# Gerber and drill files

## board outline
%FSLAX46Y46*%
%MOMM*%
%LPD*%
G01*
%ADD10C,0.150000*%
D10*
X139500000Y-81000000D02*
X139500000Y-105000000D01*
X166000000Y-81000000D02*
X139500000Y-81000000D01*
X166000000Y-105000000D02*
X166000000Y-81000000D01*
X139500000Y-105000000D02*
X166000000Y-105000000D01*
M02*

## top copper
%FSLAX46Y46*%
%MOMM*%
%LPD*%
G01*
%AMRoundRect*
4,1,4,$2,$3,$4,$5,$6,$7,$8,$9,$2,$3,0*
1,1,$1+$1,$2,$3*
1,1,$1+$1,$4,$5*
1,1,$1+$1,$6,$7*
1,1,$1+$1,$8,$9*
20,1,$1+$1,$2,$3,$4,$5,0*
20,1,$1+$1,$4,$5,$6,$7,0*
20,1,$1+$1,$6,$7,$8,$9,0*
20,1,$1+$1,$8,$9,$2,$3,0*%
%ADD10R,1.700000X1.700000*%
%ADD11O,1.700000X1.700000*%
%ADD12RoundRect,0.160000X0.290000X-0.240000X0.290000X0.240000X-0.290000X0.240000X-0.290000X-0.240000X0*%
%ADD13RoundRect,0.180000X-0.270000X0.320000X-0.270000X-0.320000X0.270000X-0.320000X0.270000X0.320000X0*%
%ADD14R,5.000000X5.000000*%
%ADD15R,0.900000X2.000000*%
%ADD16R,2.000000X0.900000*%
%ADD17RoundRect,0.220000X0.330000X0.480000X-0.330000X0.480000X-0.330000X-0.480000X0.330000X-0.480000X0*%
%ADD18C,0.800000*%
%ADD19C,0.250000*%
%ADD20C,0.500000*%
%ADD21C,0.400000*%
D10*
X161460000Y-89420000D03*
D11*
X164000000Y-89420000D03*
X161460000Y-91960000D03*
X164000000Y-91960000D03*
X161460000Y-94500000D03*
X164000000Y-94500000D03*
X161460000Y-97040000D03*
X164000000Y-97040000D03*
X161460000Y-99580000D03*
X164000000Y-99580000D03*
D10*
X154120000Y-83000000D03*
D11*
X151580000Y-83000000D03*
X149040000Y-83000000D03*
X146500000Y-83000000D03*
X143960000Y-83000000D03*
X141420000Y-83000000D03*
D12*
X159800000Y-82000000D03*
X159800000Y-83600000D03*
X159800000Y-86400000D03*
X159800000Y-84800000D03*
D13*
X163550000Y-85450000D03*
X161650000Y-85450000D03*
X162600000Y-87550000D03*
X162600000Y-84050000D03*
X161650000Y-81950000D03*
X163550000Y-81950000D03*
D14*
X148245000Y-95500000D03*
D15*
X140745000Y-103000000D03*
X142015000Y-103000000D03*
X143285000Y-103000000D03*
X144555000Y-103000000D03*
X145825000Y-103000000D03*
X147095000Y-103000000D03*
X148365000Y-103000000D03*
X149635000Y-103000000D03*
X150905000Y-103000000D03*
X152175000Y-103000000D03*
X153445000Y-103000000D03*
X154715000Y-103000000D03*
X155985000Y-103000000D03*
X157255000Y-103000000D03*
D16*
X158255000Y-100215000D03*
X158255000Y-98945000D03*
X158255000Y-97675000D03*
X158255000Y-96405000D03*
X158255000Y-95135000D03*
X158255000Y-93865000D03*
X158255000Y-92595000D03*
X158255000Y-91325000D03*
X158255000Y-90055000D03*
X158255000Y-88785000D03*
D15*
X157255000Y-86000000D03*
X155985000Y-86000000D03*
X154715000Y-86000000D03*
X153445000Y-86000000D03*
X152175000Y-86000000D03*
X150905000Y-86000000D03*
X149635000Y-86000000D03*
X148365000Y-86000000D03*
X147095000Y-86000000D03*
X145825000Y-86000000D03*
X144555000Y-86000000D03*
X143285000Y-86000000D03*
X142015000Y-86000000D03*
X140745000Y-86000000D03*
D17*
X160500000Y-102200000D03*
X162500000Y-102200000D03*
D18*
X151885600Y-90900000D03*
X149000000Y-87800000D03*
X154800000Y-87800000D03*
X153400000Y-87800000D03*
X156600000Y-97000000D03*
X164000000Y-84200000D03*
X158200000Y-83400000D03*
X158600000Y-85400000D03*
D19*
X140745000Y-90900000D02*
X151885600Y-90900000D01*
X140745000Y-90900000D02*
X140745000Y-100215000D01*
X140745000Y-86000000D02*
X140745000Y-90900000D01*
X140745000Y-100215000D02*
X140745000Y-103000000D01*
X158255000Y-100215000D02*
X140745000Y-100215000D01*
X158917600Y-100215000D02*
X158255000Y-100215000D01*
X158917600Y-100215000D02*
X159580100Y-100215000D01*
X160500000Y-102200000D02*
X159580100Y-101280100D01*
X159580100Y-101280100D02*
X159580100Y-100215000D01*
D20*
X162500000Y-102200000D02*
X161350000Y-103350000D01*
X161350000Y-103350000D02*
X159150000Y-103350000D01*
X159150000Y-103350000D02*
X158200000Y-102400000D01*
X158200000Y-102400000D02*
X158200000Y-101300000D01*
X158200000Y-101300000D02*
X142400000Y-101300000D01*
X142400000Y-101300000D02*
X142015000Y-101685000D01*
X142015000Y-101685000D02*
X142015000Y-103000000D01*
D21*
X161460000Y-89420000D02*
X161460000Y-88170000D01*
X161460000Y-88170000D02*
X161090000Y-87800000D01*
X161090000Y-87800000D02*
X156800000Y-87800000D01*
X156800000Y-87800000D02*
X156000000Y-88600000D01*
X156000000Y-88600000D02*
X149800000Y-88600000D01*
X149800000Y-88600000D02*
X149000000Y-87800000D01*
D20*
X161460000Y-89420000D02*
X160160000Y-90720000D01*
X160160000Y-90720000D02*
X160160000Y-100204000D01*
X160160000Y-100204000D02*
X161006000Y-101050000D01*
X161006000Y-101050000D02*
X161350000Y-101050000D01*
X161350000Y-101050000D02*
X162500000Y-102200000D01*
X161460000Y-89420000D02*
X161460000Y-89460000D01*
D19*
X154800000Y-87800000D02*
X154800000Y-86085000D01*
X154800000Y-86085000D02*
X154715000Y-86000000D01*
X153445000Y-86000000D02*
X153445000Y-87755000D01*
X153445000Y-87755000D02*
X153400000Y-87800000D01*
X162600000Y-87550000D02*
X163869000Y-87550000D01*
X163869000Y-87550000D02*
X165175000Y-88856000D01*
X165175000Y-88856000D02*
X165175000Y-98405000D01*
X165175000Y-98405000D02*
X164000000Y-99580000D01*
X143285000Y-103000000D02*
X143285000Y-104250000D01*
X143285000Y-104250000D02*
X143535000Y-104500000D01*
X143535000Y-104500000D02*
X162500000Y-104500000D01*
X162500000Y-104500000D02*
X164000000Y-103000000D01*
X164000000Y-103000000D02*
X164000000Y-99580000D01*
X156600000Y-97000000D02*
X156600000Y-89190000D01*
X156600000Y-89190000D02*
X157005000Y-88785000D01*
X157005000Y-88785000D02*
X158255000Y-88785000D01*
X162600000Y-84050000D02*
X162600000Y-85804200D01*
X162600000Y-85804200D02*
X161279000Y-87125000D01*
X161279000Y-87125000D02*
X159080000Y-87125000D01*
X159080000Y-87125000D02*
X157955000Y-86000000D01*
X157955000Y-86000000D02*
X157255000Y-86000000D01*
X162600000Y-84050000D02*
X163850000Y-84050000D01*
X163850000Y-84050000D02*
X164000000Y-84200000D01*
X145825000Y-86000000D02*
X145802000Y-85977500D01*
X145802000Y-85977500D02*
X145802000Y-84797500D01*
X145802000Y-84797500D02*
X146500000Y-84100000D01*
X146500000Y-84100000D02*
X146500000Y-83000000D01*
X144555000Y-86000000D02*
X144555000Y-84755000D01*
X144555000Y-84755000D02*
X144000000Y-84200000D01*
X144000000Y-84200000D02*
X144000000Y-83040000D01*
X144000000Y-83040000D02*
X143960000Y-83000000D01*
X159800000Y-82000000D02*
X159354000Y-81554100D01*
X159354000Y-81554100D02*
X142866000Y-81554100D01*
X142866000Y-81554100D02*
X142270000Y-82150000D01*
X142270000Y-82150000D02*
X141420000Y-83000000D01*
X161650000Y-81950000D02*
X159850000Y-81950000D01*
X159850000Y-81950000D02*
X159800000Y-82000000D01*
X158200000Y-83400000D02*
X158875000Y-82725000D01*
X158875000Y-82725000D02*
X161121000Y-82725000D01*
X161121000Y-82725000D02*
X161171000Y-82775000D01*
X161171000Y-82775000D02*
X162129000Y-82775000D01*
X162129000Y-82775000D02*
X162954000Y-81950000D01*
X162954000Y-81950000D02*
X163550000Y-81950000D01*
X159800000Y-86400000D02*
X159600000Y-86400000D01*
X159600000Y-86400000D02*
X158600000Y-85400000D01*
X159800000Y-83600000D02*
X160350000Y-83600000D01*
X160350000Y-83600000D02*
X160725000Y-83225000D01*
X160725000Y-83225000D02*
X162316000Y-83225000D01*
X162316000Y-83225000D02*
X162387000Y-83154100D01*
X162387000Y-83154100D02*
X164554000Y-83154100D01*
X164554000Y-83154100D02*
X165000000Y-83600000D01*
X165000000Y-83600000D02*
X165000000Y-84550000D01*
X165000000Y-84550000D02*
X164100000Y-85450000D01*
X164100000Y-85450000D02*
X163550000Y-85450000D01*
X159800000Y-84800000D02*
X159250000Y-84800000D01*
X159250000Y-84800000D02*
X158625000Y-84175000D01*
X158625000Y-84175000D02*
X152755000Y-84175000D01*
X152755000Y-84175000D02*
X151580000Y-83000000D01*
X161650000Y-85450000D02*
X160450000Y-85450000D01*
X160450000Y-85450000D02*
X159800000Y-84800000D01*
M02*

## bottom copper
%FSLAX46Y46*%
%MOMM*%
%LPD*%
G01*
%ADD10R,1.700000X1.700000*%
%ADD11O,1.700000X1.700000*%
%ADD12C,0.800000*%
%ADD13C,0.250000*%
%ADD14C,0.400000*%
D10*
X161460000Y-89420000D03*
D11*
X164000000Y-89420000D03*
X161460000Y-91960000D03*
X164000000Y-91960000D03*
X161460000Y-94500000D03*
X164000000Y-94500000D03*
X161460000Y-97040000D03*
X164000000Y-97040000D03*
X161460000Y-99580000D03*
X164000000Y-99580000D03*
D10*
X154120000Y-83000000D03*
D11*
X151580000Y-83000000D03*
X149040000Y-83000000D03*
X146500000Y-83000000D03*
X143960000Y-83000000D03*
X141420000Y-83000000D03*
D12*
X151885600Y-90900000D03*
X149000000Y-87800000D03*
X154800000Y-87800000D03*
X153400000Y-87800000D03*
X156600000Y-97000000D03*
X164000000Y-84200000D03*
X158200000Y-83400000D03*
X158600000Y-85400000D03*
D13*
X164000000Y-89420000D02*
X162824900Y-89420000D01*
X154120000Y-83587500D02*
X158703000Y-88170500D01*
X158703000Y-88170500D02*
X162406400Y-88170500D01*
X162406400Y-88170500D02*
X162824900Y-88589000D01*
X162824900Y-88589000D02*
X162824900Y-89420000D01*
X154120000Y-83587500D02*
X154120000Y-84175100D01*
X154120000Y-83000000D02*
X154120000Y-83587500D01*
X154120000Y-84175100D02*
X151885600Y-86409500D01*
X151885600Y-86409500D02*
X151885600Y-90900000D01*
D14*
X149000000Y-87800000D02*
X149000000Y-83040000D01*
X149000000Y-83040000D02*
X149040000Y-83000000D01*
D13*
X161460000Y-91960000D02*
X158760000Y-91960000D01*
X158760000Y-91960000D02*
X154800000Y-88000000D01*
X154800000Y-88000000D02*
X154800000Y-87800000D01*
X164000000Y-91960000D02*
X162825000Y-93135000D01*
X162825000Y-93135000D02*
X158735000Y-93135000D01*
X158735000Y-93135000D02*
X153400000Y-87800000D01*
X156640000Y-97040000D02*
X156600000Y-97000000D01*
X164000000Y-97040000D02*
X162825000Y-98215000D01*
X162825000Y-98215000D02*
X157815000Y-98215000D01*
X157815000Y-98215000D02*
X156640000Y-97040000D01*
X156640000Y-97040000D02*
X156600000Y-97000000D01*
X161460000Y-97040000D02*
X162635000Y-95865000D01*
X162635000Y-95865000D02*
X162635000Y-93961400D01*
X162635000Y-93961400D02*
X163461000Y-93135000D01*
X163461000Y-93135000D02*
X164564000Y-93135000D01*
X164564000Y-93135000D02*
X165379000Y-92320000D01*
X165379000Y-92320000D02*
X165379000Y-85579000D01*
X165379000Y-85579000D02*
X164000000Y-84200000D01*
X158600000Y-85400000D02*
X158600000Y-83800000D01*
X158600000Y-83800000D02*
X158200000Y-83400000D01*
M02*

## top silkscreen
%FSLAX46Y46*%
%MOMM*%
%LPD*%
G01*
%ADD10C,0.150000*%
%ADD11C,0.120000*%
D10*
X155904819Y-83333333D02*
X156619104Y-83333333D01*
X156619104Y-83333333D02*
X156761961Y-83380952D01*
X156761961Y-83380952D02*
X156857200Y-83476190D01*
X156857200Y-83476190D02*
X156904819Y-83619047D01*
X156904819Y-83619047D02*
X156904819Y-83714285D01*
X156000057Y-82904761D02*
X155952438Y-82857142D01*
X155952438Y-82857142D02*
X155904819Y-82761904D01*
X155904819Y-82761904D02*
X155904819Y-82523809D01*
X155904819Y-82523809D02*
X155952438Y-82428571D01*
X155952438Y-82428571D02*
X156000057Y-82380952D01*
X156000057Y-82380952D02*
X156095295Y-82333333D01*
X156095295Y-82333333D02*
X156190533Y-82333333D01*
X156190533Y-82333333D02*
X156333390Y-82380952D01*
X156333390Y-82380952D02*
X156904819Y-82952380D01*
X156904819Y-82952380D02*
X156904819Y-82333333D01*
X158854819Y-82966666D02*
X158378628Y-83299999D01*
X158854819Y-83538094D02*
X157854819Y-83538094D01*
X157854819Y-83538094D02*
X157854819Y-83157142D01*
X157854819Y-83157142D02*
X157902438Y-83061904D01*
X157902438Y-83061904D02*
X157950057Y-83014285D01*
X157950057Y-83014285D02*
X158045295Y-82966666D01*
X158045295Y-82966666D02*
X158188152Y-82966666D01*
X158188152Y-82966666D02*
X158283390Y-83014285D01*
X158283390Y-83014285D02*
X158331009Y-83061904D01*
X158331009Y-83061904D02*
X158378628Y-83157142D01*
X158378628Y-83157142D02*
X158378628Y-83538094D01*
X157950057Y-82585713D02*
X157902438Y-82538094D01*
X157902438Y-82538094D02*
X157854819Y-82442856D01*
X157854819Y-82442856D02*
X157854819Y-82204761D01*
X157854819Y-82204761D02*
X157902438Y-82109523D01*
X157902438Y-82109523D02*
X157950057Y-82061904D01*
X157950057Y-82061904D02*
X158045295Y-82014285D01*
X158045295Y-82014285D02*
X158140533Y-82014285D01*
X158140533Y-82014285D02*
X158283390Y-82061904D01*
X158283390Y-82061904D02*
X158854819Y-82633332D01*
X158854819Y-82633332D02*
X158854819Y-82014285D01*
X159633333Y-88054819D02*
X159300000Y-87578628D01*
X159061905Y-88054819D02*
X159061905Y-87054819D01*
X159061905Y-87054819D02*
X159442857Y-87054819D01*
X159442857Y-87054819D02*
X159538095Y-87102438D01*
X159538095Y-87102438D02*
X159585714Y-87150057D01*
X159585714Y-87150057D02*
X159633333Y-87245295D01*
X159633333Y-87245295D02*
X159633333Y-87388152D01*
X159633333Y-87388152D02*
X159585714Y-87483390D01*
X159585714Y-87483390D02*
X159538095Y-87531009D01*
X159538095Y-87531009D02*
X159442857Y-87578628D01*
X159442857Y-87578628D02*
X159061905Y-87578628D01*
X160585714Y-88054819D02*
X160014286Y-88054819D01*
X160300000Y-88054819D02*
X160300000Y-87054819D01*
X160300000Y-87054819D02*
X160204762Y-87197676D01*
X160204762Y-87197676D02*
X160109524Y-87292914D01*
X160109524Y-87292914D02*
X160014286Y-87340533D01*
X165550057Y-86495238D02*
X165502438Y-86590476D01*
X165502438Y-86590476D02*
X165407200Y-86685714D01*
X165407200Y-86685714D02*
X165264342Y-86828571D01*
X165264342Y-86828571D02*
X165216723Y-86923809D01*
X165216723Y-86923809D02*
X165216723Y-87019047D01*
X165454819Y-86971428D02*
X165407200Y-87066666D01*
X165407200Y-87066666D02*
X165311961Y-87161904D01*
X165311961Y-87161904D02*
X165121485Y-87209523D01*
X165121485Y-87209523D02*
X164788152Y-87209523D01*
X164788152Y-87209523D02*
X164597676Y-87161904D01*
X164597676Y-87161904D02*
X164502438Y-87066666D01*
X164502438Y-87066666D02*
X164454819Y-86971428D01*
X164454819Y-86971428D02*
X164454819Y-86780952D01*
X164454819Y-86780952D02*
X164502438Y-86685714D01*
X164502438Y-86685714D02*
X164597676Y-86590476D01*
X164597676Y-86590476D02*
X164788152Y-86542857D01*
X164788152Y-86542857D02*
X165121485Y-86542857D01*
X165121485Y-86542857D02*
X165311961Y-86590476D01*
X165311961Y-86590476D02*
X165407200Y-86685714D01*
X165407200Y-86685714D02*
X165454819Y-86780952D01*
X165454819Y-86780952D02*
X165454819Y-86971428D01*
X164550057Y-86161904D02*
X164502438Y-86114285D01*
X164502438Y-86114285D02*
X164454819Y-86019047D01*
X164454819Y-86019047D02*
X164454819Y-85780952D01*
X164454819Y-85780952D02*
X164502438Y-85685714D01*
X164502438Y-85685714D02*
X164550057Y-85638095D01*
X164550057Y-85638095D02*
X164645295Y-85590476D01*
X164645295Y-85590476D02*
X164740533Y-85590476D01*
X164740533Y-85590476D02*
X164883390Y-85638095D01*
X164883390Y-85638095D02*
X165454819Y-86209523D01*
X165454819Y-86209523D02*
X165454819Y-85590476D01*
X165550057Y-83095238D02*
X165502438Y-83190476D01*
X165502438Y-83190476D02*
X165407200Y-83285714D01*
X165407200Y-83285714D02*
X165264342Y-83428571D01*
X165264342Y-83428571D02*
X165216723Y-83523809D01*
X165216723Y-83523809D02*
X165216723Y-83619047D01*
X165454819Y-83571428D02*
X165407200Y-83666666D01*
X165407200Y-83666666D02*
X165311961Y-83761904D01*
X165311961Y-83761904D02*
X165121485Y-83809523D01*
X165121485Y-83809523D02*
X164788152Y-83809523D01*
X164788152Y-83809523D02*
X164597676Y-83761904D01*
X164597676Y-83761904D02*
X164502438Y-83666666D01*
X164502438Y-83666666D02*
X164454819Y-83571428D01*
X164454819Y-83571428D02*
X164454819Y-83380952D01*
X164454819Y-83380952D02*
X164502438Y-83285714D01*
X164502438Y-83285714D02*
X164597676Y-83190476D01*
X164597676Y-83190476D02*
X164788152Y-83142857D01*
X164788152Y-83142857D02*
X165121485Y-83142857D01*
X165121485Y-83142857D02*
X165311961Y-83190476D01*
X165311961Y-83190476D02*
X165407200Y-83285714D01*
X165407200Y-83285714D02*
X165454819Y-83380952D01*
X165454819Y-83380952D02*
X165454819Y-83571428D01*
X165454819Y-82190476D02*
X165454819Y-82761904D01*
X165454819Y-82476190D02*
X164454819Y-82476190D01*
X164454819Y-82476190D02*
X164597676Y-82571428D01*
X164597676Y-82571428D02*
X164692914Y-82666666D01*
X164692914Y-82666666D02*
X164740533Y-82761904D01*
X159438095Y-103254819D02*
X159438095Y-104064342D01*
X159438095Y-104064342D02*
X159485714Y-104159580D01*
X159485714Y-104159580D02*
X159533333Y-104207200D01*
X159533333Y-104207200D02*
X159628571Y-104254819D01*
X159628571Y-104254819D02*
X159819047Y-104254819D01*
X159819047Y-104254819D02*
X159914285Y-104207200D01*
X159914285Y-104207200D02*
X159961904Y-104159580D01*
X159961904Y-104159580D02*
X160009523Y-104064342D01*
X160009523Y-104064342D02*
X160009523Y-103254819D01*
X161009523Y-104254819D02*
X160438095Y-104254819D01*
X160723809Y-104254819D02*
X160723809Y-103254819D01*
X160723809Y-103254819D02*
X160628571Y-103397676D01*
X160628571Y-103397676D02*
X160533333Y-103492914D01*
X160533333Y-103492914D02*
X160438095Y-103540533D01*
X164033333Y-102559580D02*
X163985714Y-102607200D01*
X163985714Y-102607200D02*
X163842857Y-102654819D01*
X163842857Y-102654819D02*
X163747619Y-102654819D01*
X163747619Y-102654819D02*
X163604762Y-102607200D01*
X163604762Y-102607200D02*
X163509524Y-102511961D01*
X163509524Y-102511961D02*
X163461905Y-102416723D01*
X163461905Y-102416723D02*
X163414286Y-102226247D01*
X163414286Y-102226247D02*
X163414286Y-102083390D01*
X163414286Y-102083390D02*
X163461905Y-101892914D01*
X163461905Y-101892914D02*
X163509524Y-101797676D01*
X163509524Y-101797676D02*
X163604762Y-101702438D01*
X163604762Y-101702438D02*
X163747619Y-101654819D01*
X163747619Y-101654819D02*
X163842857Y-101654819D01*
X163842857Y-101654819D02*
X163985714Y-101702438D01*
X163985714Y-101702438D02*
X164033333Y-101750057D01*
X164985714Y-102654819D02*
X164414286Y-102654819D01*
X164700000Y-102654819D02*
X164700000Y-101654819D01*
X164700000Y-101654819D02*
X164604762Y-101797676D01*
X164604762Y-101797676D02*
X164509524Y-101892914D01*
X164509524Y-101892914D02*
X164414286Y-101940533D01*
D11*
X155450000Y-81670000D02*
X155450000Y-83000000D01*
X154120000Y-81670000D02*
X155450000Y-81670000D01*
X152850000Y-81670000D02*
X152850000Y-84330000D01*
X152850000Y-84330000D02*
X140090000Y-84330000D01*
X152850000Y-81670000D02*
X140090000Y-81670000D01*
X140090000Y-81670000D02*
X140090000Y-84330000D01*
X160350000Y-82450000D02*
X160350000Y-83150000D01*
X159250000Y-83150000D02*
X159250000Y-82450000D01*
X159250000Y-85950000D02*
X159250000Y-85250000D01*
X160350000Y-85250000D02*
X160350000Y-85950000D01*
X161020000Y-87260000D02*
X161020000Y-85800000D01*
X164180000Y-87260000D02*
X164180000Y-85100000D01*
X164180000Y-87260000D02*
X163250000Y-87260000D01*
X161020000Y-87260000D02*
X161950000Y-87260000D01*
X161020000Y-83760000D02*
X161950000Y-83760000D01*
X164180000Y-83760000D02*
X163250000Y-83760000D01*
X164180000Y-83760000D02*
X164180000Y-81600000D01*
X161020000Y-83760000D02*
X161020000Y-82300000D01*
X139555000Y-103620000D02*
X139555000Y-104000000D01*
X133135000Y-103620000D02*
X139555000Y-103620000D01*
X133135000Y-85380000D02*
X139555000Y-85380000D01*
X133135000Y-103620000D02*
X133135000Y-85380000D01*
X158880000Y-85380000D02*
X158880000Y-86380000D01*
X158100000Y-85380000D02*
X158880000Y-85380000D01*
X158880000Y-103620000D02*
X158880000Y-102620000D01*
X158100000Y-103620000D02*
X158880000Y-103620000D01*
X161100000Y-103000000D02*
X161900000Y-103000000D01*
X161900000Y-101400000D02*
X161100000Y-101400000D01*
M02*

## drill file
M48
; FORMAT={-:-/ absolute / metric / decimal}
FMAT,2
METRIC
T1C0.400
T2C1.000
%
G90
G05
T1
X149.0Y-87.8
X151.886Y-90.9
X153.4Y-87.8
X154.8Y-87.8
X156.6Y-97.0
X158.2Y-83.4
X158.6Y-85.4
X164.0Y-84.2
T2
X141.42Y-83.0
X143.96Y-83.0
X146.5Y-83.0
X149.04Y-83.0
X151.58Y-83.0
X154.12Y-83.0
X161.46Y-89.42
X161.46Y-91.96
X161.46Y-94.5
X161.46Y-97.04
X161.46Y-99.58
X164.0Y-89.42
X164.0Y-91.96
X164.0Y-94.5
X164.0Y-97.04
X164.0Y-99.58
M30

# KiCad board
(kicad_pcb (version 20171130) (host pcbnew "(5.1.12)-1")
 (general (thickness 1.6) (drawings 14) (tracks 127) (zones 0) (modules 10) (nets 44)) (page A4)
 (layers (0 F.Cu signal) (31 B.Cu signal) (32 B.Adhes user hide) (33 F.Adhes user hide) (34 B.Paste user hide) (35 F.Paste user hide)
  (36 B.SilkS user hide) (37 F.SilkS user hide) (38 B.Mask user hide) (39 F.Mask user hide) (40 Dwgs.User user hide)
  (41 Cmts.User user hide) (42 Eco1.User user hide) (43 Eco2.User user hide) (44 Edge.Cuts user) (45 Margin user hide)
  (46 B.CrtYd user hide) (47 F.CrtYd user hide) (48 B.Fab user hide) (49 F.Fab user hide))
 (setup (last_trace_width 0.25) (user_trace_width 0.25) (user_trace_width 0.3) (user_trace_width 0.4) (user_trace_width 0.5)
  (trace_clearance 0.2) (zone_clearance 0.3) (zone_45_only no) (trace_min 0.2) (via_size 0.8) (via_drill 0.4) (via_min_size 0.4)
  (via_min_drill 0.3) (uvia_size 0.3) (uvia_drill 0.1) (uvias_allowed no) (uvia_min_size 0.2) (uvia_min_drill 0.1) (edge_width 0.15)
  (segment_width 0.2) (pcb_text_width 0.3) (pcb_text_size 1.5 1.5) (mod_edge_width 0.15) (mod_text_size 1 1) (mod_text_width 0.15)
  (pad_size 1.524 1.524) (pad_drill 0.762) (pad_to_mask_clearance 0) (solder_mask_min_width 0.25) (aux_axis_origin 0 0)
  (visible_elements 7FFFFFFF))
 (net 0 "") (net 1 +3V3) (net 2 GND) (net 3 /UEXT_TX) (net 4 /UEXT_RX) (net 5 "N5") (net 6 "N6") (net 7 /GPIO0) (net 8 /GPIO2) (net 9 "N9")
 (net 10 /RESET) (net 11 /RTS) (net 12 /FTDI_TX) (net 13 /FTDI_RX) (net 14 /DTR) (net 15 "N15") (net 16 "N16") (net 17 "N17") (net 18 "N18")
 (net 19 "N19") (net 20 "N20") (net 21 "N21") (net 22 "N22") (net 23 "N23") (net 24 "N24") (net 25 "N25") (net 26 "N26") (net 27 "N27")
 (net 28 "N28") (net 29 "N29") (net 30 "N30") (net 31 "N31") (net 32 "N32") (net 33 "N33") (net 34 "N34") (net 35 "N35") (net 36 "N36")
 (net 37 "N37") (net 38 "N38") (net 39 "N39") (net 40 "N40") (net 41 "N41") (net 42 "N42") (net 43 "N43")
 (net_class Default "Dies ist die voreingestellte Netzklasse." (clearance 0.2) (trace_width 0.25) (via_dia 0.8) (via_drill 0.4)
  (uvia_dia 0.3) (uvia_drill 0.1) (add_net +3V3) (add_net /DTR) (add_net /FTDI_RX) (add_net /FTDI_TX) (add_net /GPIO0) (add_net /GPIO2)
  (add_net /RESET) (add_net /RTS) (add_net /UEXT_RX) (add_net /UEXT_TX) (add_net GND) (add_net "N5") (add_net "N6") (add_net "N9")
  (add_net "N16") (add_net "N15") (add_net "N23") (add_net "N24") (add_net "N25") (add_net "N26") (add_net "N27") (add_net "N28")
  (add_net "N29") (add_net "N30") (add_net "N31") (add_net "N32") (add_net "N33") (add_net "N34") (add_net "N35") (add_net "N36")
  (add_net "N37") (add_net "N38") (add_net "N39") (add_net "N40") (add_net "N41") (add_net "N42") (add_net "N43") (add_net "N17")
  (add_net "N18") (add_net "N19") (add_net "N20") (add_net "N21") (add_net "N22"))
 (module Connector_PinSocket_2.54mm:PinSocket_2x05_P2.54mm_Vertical (layer B.Cu) (at 161.46 89.42 180)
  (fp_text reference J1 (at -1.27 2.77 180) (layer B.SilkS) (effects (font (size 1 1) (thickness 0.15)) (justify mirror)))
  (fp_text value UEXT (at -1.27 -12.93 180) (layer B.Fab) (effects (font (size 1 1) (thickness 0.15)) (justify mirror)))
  (pad 1 thru_hole rect (at 0 0 180) (size 1.7 1.7) (drill 1) (layers *.Cu *.Mask) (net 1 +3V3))
  (pad 2 thru_hole oval (at -2.54 0 180) (size 1.7 1.7) (drill 1) (layers *.Cu *.Mask) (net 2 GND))
  (pad 3 thru_hole oval (at 0 -2.54 180) (size 1.7 1.7) (drill 1) (layers *.Cu *.Mask) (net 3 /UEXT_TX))
  (pad 4 thru_hole oval (at -2.54 -2.54 180) (size 1.7 1.7) (drill 1) (layers *.Cu *.Mask) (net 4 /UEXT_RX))
  (pad 5 thru_hole oval (at 0 -5.08 180) (size 1.7 1.7) (drill 1) (layers *.Cu *.Mask) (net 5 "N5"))
  (pad 6 thru_hole oval (at -2.54 -5.08 180) (size 1.7 1.7) (drill 1) (layers *.Cu *.Mask) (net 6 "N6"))
  (pad 7 thru_hole oval (at 0 -7.62 180) (size 1.7 1.7) (drill 1) (layers *.Cu *.Mask) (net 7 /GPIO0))
  (pad 8 thru_hole oval (at -2.54 -7.62 180) (size 1.7 1.7) (drill 1) (layers *.Cu *.Mask) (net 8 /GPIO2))
  (pad 9 thru_hole oval (at 0 -10.16 180) (size 1.7 1.7) (drill 1) (layers *.Cu *.Mask) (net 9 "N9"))
  (pad 10 thru_hole oval (at -2.54 -10.16 180) (size 1.7 1.7) (drill 1) (layers *.Cu *.Mask) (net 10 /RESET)))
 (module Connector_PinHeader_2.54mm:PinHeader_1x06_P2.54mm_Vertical (layer F.Cu) (at 154.12 83 270)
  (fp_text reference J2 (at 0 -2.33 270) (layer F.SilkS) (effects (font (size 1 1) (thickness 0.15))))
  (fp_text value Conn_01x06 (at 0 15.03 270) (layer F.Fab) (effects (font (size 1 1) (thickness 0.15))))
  (fp_line (start -1.33 -1.33) (end 0 -1.33) (layer F.SilkS) (width 0.12))
  (fp_line (start -1.33 0) (end -1.33 -1.33) (layer F.SilkS) (width 0.12))
  (fp_line (start -1.33 1.27) (end 1.33 1.27) (layer F.SilkS) (width 0.12))
  (fp_line (start 1.33 1.27) (end 1.33 14.03) (layer F.SilkS) (width 0.12))
  (fp_line (start -1.33 1.27) (end -1.33 14.03) (layer F.SilkS) (width 0.12))
  (fp_line (start -1.33 14.03) (end 1.33 14.03) (layer F.SilkS) (width 0.12))
  (pad 1 thru_hole rect (at 0 0 270) (size 1.7 1.7) (drill 1) (layers *.Cu *.Mask) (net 2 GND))
  (pad 2 thru_hole oval (at 0 2.54 270) (size 1.7 1.7) (drill 1) (layers *.Cu *.Mask) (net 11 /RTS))
  (pad 3 thru_hole oval (at 0 5.08 270) (size 1.7 1.7) (drill 1) (layers *.Cu *.Mask) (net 1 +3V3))
  (pad 4 thru_hole oval (at 0 7.62 270) (size 1.7 1.7) (drill 1) (layers *.Cu *.Mask) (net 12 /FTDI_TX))
  (pad 5 thru_hole oval (at 0 10.16 270) (size 1.7 1.7) (drill 1) (layers *.Cu *.Mask) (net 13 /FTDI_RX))
  (pad 6 thru_hole oval (at 0 12.7 270) (size 1.7 1.7) (drill 1) (layers *.Cu *.Mask) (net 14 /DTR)))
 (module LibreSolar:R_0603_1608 (layer F.Cu) (at 159.8 82.8 90)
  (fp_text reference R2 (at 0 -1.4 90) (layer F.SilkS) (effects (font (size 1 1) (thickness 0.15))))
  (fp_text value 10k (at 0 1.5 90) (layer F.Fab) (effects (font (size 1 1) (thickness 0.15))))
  (fp_line (start 0.35 0.55) (end -0.35 0.55) (layer F.SilkS) (width 0.12))
  (fp_line (start -0.35 -0.55) (end 0.35 -0.55) (layer F.SilkS) (width 0.12))
  (pad 2 smd roundrect (at 0.8 0 90) (size 0.8 0.9) (layers F.Cu F.Paste F.Mask) (roundrect_rratio 0.2) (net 14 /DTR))
  (pad 1 smd roundrect (at -0.8 0 90) (size 0.8 0.9) (layers F.Cu F.Paste F.Mask) (roundrect_rratio 0.2) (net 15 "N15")))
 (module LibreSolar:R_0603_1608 (layer F.Cu) (at 159.8 85.6 90)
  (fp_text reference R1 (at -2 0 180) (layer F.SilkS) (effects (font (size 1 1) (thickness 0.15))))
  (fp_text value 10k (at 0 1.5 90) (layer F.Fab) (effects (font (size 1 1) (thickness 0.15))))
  (fp_line (start -0.35 -0.55) (end 0.35 -0.55) (layer F.SilkS) (width 0.12))
  (fp_line (start 0.35 0.55) (end -0.35 0.55) (layer F.SilkS) (width 0.12))
  (pad 1 smd roundrect (at -0.8 0 90) (size 0.8 0.9) (layers F.Cu F.Paste F.Mask) (roundrect_rratio 0.2) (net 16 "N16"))
  (pad 2 smd roundrect (at 0.8 0 90) (size 0.8 0.9) (layers F.Cu F.Paste F.Mask) (roundrect_rratio 0.2) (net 11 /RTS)))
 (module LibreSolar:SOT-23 (layer F.Cu) (at 162.6 86.5 270)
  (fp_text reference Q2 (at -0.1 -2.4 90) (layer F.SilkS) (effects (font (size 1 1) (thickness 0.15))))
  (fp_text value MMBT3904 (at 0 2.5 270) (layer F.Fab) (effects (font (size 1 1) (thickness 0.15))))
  (fp_line (start 0.76 1.58) (end -0.7 1.58) (layer F.SilkS) (width 0.12))
  (fp_line (start 0.76 -1.58) (end -1.4 -1.58) (layer F.SilkS) (width 0.12))
  (fp_line (start 0.76 -1.58) (end 0.76 -0.65) (layer F.SilkS) (width 0.12))
  (fp_line (start 0.76 1.58) (end 0.76 0.65) (layer F.SilkS) (width 0.12))
  (pad 1 smd roundrect (at -1.05 -0.95 270) (size 1 0.9) (layers F.Cu F.Paste F.Mask) (roundrect_rratio 0.2) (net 15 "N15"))
  (pad 2 smd roundrect (at -1.05 0.95 270) (size 1 0.9) (layers F.Cu F.Paste F.Mask) (roundrect_rratio 0.2) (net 11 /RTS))
  (pad 3 smd roundrect (at 1.05 0 270) (size 1 0.9) (layers F.Cu F.Paste F.Mask) (roundrect_rratio 0.2) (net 10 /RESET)))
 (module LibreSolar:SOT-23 (layer F.Cu) (at 162.6 83 270)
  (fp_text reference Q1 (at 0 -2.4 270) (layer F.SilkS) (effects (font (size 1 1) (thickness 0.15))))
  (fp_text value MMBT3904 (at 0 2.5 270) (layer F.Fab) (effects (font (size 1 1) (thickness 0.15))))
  (fp_line (start 0.76 1.58) (end 0.76 0.65) (layer F.SilkS) (width 0.12))
  (fp_line (start 0.76 -1.58) (end 0.76 -0.65) (layer F.SilkS) (width 0.12))
  (fp_line (start 0.76 -1.58) (end -1.4 -1.58) (layer F.SilkS) (width 0.12))
  (fp_line (start 0.76 1.58) (end -0.7 1.58) (layer F.SilkS) (width 0.12))
  (pad 3 smd roundrect (at 1.05 0 270) (size 1 0.9) (layers F.Cu F.Paste F.Mask) (roundrect_rratio 0.2) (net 7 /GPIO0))
  (pad 2 smd roundrect (at -1.05 0.95 270) (size 1 0.9) (layers F.Cu F.Paste F.Mask) (roundrect_rratio 0.2) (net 14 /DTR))
  (pad 1 smd roundrect (at -1.05 -0.95 270) (size 1 0.9) (layers F.Cu F.Paste F.Mask) (roundrect_rratio 0.2) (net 16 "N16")))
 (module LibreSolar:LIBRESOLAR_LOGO (layer B.Cu) (at 156 98 180)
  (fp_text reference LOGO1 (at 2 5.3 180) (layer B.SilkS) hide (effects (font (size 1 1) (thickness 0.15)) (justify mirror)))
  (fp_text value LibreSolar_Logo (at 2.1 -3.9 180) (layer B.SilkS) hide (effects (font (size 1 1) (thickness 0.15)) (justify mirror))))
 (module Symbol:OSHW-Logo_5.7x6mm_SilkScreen (layer B.Cu) (at 145.4 97 180)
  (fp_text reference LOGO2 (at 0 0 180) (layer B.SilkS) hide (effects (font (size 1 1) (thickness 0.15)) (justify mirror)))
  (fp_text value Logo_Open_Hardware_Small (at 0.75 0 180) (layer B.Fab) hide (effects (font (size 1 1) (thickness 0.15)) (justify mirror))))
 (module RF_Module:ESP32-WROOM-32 (layer F.Cu) (at 149 94.5 90)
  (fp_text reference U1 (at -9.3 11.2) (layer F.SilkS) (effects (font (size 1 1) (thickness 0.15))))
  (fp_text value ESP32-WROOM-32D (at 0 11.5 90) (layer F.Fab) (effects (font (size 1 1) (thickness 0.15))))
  (fp_line (start -9.12 -9.445) (end -9.5 -9.445) (layer F.SilkS) (width 0.12))
  (fp_line (start -9.12 -15.865) (end -9.12 -9.445) (layer F.SilkS) (width 0.12))
  (fp_line (start 9.12 -15.865) (end 9.12 -9.445) (layer F.SilkS) (width 0.12))
  (fp_line (start -9.12 -15.865) (end 9.12 -15.865) (layer F.SilkS) (width 0.12))
  (fp_line (start 9.12 9.88) (end 8.12 9.88) (layer F.SilkS) (width 0.12))
  (fp_line (start 9.12 9.1) (end 9.12 9.88) (layer F.SilkS) (width 0.12))
  (fp_line (start -9.12 9.88) (end -8.12 9.88) (layer F.SilkS) (width 0.12))
  (fp_line (start -9.12 9.1) (end -9.12 9.88) (layer F.SilkS) (width 0.12))
  (pad 39 smd rect (at -1 -0.755 90) (size 5 5) (layers F.Cu F.Paste F.Mask))
  (pad 1 smd rect (at -8.5 -8.255 90) (size 2 0.9) (layers F.Cu F.Paste F.Mask) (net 2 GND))
  (pad 2 smd rect (at -8.5 -6.985 90) (size 2 0.9) (layers F.Cu F.Paste F.Mask) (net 1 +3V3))
  (pad 3 smd rect (at -8.5 -5.715 90) (size 2 0.9) (layers F.Cu F.Paste F.Mask) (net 10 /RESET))
  (pad 4 smd rect (at -8.5 -4.445 90) (size 2 0.9) (layers F.Cu F.Paste F.Mask) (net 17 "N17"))
  (pad 5 smd rect (at -8.5 -3.175 90) (size 2 0.9) (layers F.Cu F.Paste F.Mask) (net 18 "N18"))
  (pad 6 smd rect (at -8.5 -1.905 90) (size 2 0.9) (layers F.Cu F.Paste F.Mask) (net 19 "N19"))
  (pad 7 smd rect (at -8.5 -0.635 90) (size 2 0.9) (layers F.Cu F.Paste F.Mask) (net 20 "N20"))
  (pad 8 smd rect (at -8.5 0.635 90) (size 2 0.9) (layers F.Cu F.Paste F.Mask) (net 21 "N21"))
  (pad 9 smd rect (at -8.5 1.905 90) (size 2 0.9) (layers F.Cu F.Paste F.Mask) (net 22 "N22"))
  (pad 10 smd rect (at -8.5 3.175 90) (size 2 0.9) (layers F.Cu F.Paste F.Mask) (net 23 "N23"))
  (pad 11 smd rect (at -8.5 4.445 90) (size 2 0.9) (layers F.Cu F.Paste F.Mask) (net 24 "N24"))
  (pad 12 smd rect (at -8.5 5.715 90) (size 2 0.9) (layers F.Cu F.Paste F.Mask) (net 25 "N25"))
  (pad 13 smd rect (at -8.5 6.985 90) (size 2 0.9) (layers F.Cu F.Paste F.Mask) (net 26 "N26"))
  (pad 14 smd rect (at -8.5 8.255 90) (size 2 0.9) (layers F.Cu F.Paste F.Mask) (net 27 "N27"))
  (pad 15 smd rect (at -5.715 9.255 180) (size 2 0.9) (layers F.Cu F.Paste F.Mask) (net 2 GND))
  (pad 16 smd rect (at -4.445 9.255 180) (size 2 0.9) (layers F.Cu F.Paste F.Mask) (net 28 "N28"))
  (pad 17 smd rect (at -3.175 9.255 180) (size 2 0.9) (layers F.Cu F.Paste F.Mask) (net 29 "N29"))
  (pad 18 smd rect (at -1.905 9.255 180) (size 2 0.9) (layers F.Cu F.Paste F.Mask) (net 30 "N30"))
  (pad 19 smd rect (at -0.635 9.255 180) (size 2 0.9) (layers F.Cu F.Paste F.Mask) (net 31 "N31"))
  (pad 20 smd rect (at 0.635 9.255 180) (size 2 0.9) (layers F.Cu F.Paste F.Mask) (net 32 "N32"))
  (pad 21 smd rect (at 1.905 9.255 180) (size 2 0.9) (layers F.Cu F.Paste F.Mask) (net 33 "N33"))
  (pad 22 smd rect (at 3.175 9.255 180) (size 2 0.9) (layers F.Cu F.Paste F.Mask) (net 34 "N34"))
  (pad 23 smd rect (at 4.445 9.255 180) (size 2 0.9) (layers F.Cu F.Paste F.Mask) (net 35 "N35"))
  (pad 24 smd rect (at 5.715 9.255 180) (size 2 0.9) (layers F.Cu F.Paste F.Mask) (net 8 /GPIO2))
  (pad 25 smd rect (at 8.5 8.255 90) (size 2 0.9) (layers F.Cu F.Paste F.Mask) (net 7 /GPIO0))
  (pad 26 smd rect (at 8.5 6.985 90) (size 2 0.9) (layers F.Cu F.Paste F.Mask) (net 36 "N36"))
  (pad 27 smd rect (at 8.5 5.715 90) (size 2 0.9) (layers F.Cu F.Paste F.Mask) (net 3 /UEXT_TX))
  (pad 28 smd rect (at 8.5 4.445 90) (size 2 0.9) (layers F.Cu F.Paste F.Mask) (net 4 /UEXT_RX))
  (pad 29 smd rect (at 8.5 3.175 90) (size 2 0.9) (layers F.Cu F.Paste F.Mask) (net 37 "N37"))
  (pad 30 smd rect (at 8.5 1.905 90) (size 2 0.9) (layers F.Cu F.Paste F.Mask) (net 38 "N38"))
  (pad 31 smd rect (at 8.5 0.635 90) (size 2 0.9) (layers F.Cu F.Paste F.Mask) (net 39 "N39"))
  (pad 32 smd rect (at 8.5 -0.635 90) (size 2 0.9) (layers F.Cu F.Paste F.Mask) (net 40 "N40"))
  (pad 33 smd rect (at 8.5 -1.905 90) (size 2 0.9) (layers F.Cu F.Paste F.Mask) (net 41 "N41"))
  (pad 34 smd rect (at 8.5 -3.175 90) (size 2 0.9) (layers F.Cu F.Paste F.Mask) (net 12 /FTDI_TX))
  (pad 35 smd rect (at 8.5 -4.445 90) (size 2 0.9) (layers F.Cu F.Paste F.Mask) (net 13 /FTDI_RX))
  (pad 36 smd rect (at 8.5 -5.715 90) (size 2 0.9) (layers F.Cu F.Paste F.Mask) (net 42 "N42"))
  (pad 37 smd rect (at 8.5 -6.985 90) (size 2 0.9) (layers F.Cu F.Paste F.Mask) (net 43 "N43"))
  (pad 38 smd rect (at 8.5 -8.255 90) (size 2 0.9) (layers F.Cu F.Paste F.Mask) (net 2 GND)))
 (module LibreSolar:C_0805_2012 (layer F.Cu) (at 161.5 102.2 180)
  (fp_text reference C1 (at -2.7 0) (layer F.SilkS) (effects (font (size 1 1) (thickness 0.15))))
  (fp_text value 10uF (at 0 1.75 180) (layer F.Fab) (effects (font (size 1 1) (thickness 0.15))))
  (fp_line (start 0.4 -0.8) (end -0.4 -0.8) (layer F.SilkS) (width 0.12))
  (fp_line (start -0.4 0.8) (end 0.4 0.8) (layer F.SilkS) (width 0.12))
  (pad 2 smd roundrect (at 1 0 180) (size 1.1 1.4) (layers F.Cu F.Paste F.Mask) (roundrect_rratio 0.2) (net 2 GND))
  (pad 1 smd roundrect (at -1 0 180) (size 1.1 1.4) (layers F.Cu F.Paste F.Mask) (roundrect_rratio 0.2) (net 1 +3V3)))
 (gr_line (start 139.5 81) (end 139.5 105) (layer Edge.Cuts) (width 0.15))
 (gr_line (start 166 81) (end 139.5 81) (layer Edge.Cuts) (width 0.15))
 (gr_line (start 166 105) (end 166 81) (layer Edge.Cuts) (width 0.15))
 (gr_line (start 139.5 105) (end 166 105) (layer Edge.Cuts) (width 0.15))
 (segment (start 164 89.42) (end 162.8249 89.42) (width 0.25) (layer B.Cu) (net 2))
 (segment (start 154.12 83.5875) (end 158.703 88.1705) (width 0.25) (layer B.Cu) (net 2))
 (segment (start 158.703 88.1705) (end 162.4064 88.1705) (width 0.25) (layer B.Cu) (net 2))
 (segment (start 162.4064 88.1705) (end 162.8249 88.589) (width 0.25) (layer B.Cu) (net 2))
 (segment (start 162.8249 88.589) (end 162.8249 89.42) (width 0.25) (layer B.Cu) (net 2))
 (segment (start 154.12 83.5875) (end 154.12 84.1751) (width 0.25) (layer B.Cu) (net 2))
 (segment (start 154.12 83) (end 154.12 83.5875) (width 0.25) (layer B.Cu) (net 2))
 (segment (start 140.745 90.9) (end 151.8856 90.9) (width 0.25) (layer F.Cu) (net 2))
 (segment (start 154.12 84.1751) (end 151.8856 86.4095) (width 0.25) (layer B.Cu) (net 2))
 (segment (start 151.8856 86.4095) (end 151.8856 90.9) (width 0.25) (layer B.Cu) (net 2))
 (segment (start 140.745 90.9) (end 140.745 100.215) (width 0.25) (layer F.Cu) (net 2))
 (segment (start 140.745 86) (end 140.745 90.9) (width 0.25) (layer F.Cu) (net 2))
 (segment (start 140.745 100.215) (end 140.745 103) (width 0.25) (layer F.Cu) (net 2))
 (segment (start 158.255 100.215) (end 140.745 100.215) (width 0.25) (layer F.Cu) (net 2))
 (segment (start 158.9176 100.215) (end 158.255 100.215) (width 0.25) (layer F.Cu) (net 2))
 (segment (start 158.9176 100.215) (end 159.5801 100.215) (width 0.25) (layer F.Cu) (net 2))
 (segment (start 160.5 102.2) (end 159.5801 101.2801) (width 0.25) (layer F.Cu) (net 2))
 (segment (start 159.5801 101.2801) (end 159.5801 100.215) (width 0.25) (layer F.Cu) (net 2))
 (via (at 151.8856 90.9) (size 0.8) (layers F.Cu B.Cu) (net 2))
 (segment (start 162.5 102.2) (end 161.35 103.35) (width 0.5) (layer F.Cu) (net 1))
 (segment (start 161.35 103.35) (end 159.15 103.35) (width 0.5) (layer F.Cu) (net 1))
 (segment (start 159.15 103.35) (end 158.2 102.4) (width 0.5) (layer F.Cu) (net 1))
 (segment (start 158.2 102.4) (end 158.2 101.3) (width 0.5) (layer F.Cu) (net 1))
 (segment (start 158.2 101.3) (end 142.4 101.3) (width 0.5) (layer F.Cu) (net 1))
 (segment (start 142.4 101.3) (end 142.015 101.685) (width 0.5) (layer F.Cu) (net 1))
 (segment (start 142.015 101.685) (end 142.015 103) (width 0.5) (layer F.Cu) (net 1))
 (segment (start 161.46 89.42) (end 161.46 88.17) (width 0.4) (layer F.Cu) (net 1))
 (segment (start 161.46 88.17) (end 161.09 87.8) (width 0.4) (layer F.Cu) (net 1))
 (segment (start 161.09 87.8) (end 156.8 87.8) (width 0.4) (layer F.Cu) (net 1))
 (segment (start 156.8 87.8) (end 156 88.6) (width 0.4) (layer F.Cu) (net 1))
 (segment (start 156 88.6) (end 149.8 88.6) (width 0.4) (layer F.Cu) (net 1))
 (segment (start 149.8 88.6) (end 149 87.8) (width 0.4) (layer F.Cu) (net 1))
 (segment (start 149 87.8) (end 149 83.04) (width 0.4) (layer B.Cu) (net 1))
 (segment (start 149 83.04) (end 149.04 83) (width 0.4) (layer B.Cu) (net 1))
 (segment (start 161.46 89.42) (end 160.16 90.72) (width 0.5) (layer F.Cu) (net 1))
 (segment (start 160.16 90.72) (end 160.16 100.204) (width 0.5) (layer F.Cu) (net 1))
 (segment (start 160.16 100.204) (end 161.006 101.05) (width 0.5) (layer F.Cu) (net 1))
 (segment (start 161.006 101.05) (end 161.35 101.05) (width 0.5) (layer F.Cu) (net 1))
 (segment (start 161.35 101.05) (end 162.5 102.2) (width 0.5) (layer F.Cu) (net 1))
 (segment (start 161.46 89.42) (end 161.46 89.46) (width 0.5) (layer F.Cu) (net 1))
 (via (at 149 87.8) (size 0.8) (layers F.Cu B.Cu) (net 1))
 (segment (start 161.46 91.96) (end 158.76 91.96) (width 0.25) (layer B.Cu) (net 3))
 (segment (start 158.76 91.96) (end 154.8 88) (width 0.25) (layer B.Cu) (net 3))
 (segment (start 154.8 88) (end 154.8 87.8) (width 0.25) (layer B.Cu) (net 3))
 (segment (start 154.8 87.8) (end 154.8 86.085) (width 0.25) (layer F.Cu) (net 3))
 (segment (start 154.8 86.085) (end 154.715 86) (width 0.25) (layer F.Cu) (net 3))
 (via (at 154.8 87.8) (size 0.8) (layers F.Cu B.Cu) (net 3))
 (segment (start 164 91.96) (end 162.825 93.135) (width 0.25) (layer B.Cu) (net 4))
 (segment (start 162.825 93.135) (end 158.735 93.135) (width 0.25) (layer B.Cu) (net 4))
 (segment (start 158.735 93.135) (end 153.4 87.8) (width 0.25) (layer B.Cu) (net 4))
 (segment (start 153.445 86) (end 153.445 87.755) (width 0.25) (layer F.Cu) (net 4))
 (segment (start 153.445 87.755) (end 153.4 87.8) (width 0.25) (layer F.Cu) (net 4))
 (via (at 153.4 87.8) (size 0.8) (layers F.Cu B.Cu) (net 4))
 (segment (start 162.6 87.55) (end 163.869 87.55) (width 0.25) (layer F.Cu) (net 10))
 (segment (start 163.869 87.55) (end 165.175 88.856) (width 0.25) (layer F.Cu) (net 10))
 (segment (start 165.175 88.856) (end 165.175 98.405) (width 0.25) (layer F.Cu) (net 10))
 (segment (start 165.175 98.405) (end 164 99.58) (width 0.25) (layer F.Cu) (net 10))
 (segment (start 143.285 103) (end 143.285 104.25) (width 0.25) (layer F.Cu) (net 10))
 (segment (start 143.285 104.25) (end 143.535 104.5) (width 0.25) (layer F.Cu) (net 10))
 (segment (start 143.535 104.5) (end 162.5 104.5) (width 0.25) (layer F.Cu) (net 10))
 (segment (start 162.5 104.5) (end 164 103) (width 0.25) (layer F.Cu) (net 10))
 (segment (start 164 103) (end 164 99.58) (width 0.25) (layer F.Cu) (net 10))
 (segment (start 156.64 97.04) (end 156.6 97) (width 0.25) (layer B.Cu) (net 8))
 (segment (start 164 97.04) (end 162.825 98.215) (width 0.25) (layer B.Cu) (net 8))
 (segment (start 162.825 98.215) (end 157.815 98.215) (width 0.25) (layer B.Cu) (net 8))
 (segment (start 157.815 98.215) (end 156.64 97.04) (width 0.25) (layer B.Cu) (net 8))
 (segment (start 156.6 97) (end 156.6 89.19) (width 0.25) (layer F.Cu) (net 8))
 (segment (start 156.6 89.19) (end 157.005 88.785) (width 0.25) (layer F.Cu) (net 8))
 (segment (start 157.005 88.785) (end 158.255 88.785) (width 0.25) (layer F.Cu) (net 8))
 (segment (start 156.64 97.04) (end 156.6 97) (width 0.25) (layer B.Cu) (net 8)) (via (at 156.6 97) (size 0.8) (layers F.Cu B.Cu) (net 8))
 (segment (start 162.6 84.05) (end 162.6 85.8042) (width 0.25) (layer F.Cu) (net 7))
 (segment (start 162.6 85.8042) (end 161.279 87.125) (width 0.25) (layer F.Cu) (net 7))
 (segment (start 161.279 87.125) (end 159.08 87.125) (width 0.25) (layer F.Cu) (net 7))
 (segment (start 159.08 87.125) (end 157.955 86) (width 0.25) (layer F.Cu) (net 7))
 (segment (start 157.955 86) (end 157.255 86) (width 0.25) (layer F.Cu) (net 7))
 (segment (start 162.6 84.05) (end 163.85 84.05) (width 0.25) (layer F.Cu) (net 7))
 (segment (start 163.85 84.05) (end 164 84.2) (width 0.25) (layer F.Cu) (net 7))
 (segment (start 161.46 97.04) (end 162.635 95.865) (width 0.25) (layer B.Cu) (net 7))
 (segment (start 162.635 95.865) (end 162.635 93.9614) (width 0.25) (layer B.Cu) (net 7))
 (segment (start 162.635 93.9614) (end 163.461 93.135) (width 0.25) (layer B.Cu) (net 7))
 (segment (start 163.461 93.135) (end 164.564 93.135) (width 0.25) (layer B.Cu) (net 7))
 (segment (start 164.564 93.135) (end 165.379 92.32) (width 0.25) (layer B.Cu) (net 7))
 (segment (start 165.379 92.32) (end 165.379 85.579) (width 0.25) (layer B.Cu) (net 7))
 (segment (start 165.379 85.579) (end 164 84.2) (width 0.25) (layer B.Cu) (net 7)) (via (at 164 84.2) (size 0.8) (layers F.Cu B.Cu) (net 7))
 (segment (start 145.825 86) (end 145.802 85.9775) (width 0.25) (layer F.Cu) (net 12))
 (segment (start 145.802 85.9775) (end 145.802 84.7975) (width 0.25) (layer F.Cu) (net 12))
 (segment (start 145.802 84.7975) (end 146.5 84.1) (width 0.25) (layer F.Cu) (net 12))
 (segment (start 146.5 84.1) (end 146.5 83) (width 0.25) (layer F.Cu) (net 12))
 (segment (start 144.555 86) (end 144.555 84.755) (width 0.25) (layer F.Cu) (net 13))
 (segment (start 144.555 84.755) (end 144 84.2) (width 0.25) (layer F.Cu) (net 13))
 (segment (start 144 84.2) (end 144 83.04) (width 0.25) (layer F.Cu) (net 13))
 (segment (start 144 83.04) (end 143.96 83) (width 0.25) (layer F.Cu) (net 13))
 (segment (start 159.8 82) (end 159.354 81.5541) (width 0.25) (layer F.Cu) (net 14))
 (segment (start 159.354 81.5541) (end 142.866 81.5541) (width 0.25) (layer F.Cu) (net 14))
 (segment (start 142.866 81.5541) (end 142.27 82.15) (width 0.25) (layer F.Cu) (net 14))
 (segment (start 142.27 82.15) (end 141.42 83) (width 0.25) (layer F.Cu) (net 14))
 (segment (start 161.65 81.95) (end 159.85 81.95) (width 0.25) (layer F.Cu) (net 14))
 (segment (start 159.85 81.95) (end 159.8 82) (width 0.25) (layer F.Cu) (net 14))
 (segment (start 158.2 83.4) (end 158.875 82.725) (width 0.25) (layer F.Cu) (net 16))
 (segment (start 158.875 82.725) (end 161.121 82.725) (width 0.25) (layer F.Cu) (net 16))
 (segment (start 161.121 82.725) (end 161.171 82.775) (width 0.25) (layer F.Cu) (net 16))
 (segment (start 161.171 82.775) (end 162.129 82.775) (width 0.25) (layer F.Cu) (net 16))
 (segment (start 162.129 82.775) (end 162.954 81.95) (width 0.25) (layer F.Cu) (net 16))
 (segment (start 162.954 81.95) (end 163.55 81.95) (width 0.25) (layer F.Cu) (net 16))
 (segment (start 158.6 85.4) (end 158.6 83.8) (width 0.25) (layer B.Cu) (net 16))
 (segment (start 158.6 83.8) (end 158.2 83.4) (width 0.25) (layer B.Cu) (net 16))
 (segment (start 159.8 86.4) (end 159.6 86.4) (width 0.25) (layer F.Cu) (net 16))
 (segment (start 159.6 86.4) (end 158.6 85.4) (width 0.25) (layer F.Cu) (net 16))
 (via (at 158.2 83.4) (size 0.8) (layers F.Cu B.Cu) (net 16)) (via (at 158.6 85.4) (size 0.8) (layers F.Cu B.Cu) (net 16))
 (segment (start 159.8 83.6) (end 160.35 83.6) (width 0.25) (layer F.Cu) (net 15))
 (segment (start 160.35 83.6) (end 160.725 83.225) (width 0.25) (layer F.Cu) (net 15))
 (segment (start 160.725 83.225) (end 162.316 83.225) (width 0.25) (layer F.Cu) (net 15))
 (segment (start 162.316 83.225) (end 162.387 83.1541) (width 0.25) (layer F.Cu) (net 15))
 (segment (start 162.387 83.1541) (end 164.554 83.1541) (width 0.25) (layer F.Cu) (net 15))
 (segment (start 164.554 83.1541) (end 165 83.6) (width 0.25) (layer F.Cu) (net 15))
 (segment (start 165 83.6) (end 165 84.55) (width 0.25) (layer F.Cu) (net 15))
 (segment (start 165 84.55) (end 164.1 85.45) (width 0.25) (layer F.Cu) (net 15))
 (segment (start 164.1 85.45) (end 163.55 85.45) (width 0.25) (layer F.Cu) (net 15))
 (segment (start 159.8 84.8) (end 159.25 84.8) (width 0.25) (layer F.Cu) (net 11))
 (segment (start 159.25 84.8) (end 158.625 84.175) (width 0.25) (layer F.Cu) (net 11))
 (segment (start 158.625 84.175) (end 152.755 84.175) (width 0.25) (layer F.Cu) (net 11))
 (segment (start 152.755 84.175) (end 151.58 83) (width 0.25) (layer F.Cu) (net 11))
 (segment (start 161.65 85.45) (end 160.45 85.45) (width 0.25) (layer F.Cu) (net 11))
 (segment (start 160.45 85.45) (end 159.8 84.8) (width 0.25) (layer F.Cu) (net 11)))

